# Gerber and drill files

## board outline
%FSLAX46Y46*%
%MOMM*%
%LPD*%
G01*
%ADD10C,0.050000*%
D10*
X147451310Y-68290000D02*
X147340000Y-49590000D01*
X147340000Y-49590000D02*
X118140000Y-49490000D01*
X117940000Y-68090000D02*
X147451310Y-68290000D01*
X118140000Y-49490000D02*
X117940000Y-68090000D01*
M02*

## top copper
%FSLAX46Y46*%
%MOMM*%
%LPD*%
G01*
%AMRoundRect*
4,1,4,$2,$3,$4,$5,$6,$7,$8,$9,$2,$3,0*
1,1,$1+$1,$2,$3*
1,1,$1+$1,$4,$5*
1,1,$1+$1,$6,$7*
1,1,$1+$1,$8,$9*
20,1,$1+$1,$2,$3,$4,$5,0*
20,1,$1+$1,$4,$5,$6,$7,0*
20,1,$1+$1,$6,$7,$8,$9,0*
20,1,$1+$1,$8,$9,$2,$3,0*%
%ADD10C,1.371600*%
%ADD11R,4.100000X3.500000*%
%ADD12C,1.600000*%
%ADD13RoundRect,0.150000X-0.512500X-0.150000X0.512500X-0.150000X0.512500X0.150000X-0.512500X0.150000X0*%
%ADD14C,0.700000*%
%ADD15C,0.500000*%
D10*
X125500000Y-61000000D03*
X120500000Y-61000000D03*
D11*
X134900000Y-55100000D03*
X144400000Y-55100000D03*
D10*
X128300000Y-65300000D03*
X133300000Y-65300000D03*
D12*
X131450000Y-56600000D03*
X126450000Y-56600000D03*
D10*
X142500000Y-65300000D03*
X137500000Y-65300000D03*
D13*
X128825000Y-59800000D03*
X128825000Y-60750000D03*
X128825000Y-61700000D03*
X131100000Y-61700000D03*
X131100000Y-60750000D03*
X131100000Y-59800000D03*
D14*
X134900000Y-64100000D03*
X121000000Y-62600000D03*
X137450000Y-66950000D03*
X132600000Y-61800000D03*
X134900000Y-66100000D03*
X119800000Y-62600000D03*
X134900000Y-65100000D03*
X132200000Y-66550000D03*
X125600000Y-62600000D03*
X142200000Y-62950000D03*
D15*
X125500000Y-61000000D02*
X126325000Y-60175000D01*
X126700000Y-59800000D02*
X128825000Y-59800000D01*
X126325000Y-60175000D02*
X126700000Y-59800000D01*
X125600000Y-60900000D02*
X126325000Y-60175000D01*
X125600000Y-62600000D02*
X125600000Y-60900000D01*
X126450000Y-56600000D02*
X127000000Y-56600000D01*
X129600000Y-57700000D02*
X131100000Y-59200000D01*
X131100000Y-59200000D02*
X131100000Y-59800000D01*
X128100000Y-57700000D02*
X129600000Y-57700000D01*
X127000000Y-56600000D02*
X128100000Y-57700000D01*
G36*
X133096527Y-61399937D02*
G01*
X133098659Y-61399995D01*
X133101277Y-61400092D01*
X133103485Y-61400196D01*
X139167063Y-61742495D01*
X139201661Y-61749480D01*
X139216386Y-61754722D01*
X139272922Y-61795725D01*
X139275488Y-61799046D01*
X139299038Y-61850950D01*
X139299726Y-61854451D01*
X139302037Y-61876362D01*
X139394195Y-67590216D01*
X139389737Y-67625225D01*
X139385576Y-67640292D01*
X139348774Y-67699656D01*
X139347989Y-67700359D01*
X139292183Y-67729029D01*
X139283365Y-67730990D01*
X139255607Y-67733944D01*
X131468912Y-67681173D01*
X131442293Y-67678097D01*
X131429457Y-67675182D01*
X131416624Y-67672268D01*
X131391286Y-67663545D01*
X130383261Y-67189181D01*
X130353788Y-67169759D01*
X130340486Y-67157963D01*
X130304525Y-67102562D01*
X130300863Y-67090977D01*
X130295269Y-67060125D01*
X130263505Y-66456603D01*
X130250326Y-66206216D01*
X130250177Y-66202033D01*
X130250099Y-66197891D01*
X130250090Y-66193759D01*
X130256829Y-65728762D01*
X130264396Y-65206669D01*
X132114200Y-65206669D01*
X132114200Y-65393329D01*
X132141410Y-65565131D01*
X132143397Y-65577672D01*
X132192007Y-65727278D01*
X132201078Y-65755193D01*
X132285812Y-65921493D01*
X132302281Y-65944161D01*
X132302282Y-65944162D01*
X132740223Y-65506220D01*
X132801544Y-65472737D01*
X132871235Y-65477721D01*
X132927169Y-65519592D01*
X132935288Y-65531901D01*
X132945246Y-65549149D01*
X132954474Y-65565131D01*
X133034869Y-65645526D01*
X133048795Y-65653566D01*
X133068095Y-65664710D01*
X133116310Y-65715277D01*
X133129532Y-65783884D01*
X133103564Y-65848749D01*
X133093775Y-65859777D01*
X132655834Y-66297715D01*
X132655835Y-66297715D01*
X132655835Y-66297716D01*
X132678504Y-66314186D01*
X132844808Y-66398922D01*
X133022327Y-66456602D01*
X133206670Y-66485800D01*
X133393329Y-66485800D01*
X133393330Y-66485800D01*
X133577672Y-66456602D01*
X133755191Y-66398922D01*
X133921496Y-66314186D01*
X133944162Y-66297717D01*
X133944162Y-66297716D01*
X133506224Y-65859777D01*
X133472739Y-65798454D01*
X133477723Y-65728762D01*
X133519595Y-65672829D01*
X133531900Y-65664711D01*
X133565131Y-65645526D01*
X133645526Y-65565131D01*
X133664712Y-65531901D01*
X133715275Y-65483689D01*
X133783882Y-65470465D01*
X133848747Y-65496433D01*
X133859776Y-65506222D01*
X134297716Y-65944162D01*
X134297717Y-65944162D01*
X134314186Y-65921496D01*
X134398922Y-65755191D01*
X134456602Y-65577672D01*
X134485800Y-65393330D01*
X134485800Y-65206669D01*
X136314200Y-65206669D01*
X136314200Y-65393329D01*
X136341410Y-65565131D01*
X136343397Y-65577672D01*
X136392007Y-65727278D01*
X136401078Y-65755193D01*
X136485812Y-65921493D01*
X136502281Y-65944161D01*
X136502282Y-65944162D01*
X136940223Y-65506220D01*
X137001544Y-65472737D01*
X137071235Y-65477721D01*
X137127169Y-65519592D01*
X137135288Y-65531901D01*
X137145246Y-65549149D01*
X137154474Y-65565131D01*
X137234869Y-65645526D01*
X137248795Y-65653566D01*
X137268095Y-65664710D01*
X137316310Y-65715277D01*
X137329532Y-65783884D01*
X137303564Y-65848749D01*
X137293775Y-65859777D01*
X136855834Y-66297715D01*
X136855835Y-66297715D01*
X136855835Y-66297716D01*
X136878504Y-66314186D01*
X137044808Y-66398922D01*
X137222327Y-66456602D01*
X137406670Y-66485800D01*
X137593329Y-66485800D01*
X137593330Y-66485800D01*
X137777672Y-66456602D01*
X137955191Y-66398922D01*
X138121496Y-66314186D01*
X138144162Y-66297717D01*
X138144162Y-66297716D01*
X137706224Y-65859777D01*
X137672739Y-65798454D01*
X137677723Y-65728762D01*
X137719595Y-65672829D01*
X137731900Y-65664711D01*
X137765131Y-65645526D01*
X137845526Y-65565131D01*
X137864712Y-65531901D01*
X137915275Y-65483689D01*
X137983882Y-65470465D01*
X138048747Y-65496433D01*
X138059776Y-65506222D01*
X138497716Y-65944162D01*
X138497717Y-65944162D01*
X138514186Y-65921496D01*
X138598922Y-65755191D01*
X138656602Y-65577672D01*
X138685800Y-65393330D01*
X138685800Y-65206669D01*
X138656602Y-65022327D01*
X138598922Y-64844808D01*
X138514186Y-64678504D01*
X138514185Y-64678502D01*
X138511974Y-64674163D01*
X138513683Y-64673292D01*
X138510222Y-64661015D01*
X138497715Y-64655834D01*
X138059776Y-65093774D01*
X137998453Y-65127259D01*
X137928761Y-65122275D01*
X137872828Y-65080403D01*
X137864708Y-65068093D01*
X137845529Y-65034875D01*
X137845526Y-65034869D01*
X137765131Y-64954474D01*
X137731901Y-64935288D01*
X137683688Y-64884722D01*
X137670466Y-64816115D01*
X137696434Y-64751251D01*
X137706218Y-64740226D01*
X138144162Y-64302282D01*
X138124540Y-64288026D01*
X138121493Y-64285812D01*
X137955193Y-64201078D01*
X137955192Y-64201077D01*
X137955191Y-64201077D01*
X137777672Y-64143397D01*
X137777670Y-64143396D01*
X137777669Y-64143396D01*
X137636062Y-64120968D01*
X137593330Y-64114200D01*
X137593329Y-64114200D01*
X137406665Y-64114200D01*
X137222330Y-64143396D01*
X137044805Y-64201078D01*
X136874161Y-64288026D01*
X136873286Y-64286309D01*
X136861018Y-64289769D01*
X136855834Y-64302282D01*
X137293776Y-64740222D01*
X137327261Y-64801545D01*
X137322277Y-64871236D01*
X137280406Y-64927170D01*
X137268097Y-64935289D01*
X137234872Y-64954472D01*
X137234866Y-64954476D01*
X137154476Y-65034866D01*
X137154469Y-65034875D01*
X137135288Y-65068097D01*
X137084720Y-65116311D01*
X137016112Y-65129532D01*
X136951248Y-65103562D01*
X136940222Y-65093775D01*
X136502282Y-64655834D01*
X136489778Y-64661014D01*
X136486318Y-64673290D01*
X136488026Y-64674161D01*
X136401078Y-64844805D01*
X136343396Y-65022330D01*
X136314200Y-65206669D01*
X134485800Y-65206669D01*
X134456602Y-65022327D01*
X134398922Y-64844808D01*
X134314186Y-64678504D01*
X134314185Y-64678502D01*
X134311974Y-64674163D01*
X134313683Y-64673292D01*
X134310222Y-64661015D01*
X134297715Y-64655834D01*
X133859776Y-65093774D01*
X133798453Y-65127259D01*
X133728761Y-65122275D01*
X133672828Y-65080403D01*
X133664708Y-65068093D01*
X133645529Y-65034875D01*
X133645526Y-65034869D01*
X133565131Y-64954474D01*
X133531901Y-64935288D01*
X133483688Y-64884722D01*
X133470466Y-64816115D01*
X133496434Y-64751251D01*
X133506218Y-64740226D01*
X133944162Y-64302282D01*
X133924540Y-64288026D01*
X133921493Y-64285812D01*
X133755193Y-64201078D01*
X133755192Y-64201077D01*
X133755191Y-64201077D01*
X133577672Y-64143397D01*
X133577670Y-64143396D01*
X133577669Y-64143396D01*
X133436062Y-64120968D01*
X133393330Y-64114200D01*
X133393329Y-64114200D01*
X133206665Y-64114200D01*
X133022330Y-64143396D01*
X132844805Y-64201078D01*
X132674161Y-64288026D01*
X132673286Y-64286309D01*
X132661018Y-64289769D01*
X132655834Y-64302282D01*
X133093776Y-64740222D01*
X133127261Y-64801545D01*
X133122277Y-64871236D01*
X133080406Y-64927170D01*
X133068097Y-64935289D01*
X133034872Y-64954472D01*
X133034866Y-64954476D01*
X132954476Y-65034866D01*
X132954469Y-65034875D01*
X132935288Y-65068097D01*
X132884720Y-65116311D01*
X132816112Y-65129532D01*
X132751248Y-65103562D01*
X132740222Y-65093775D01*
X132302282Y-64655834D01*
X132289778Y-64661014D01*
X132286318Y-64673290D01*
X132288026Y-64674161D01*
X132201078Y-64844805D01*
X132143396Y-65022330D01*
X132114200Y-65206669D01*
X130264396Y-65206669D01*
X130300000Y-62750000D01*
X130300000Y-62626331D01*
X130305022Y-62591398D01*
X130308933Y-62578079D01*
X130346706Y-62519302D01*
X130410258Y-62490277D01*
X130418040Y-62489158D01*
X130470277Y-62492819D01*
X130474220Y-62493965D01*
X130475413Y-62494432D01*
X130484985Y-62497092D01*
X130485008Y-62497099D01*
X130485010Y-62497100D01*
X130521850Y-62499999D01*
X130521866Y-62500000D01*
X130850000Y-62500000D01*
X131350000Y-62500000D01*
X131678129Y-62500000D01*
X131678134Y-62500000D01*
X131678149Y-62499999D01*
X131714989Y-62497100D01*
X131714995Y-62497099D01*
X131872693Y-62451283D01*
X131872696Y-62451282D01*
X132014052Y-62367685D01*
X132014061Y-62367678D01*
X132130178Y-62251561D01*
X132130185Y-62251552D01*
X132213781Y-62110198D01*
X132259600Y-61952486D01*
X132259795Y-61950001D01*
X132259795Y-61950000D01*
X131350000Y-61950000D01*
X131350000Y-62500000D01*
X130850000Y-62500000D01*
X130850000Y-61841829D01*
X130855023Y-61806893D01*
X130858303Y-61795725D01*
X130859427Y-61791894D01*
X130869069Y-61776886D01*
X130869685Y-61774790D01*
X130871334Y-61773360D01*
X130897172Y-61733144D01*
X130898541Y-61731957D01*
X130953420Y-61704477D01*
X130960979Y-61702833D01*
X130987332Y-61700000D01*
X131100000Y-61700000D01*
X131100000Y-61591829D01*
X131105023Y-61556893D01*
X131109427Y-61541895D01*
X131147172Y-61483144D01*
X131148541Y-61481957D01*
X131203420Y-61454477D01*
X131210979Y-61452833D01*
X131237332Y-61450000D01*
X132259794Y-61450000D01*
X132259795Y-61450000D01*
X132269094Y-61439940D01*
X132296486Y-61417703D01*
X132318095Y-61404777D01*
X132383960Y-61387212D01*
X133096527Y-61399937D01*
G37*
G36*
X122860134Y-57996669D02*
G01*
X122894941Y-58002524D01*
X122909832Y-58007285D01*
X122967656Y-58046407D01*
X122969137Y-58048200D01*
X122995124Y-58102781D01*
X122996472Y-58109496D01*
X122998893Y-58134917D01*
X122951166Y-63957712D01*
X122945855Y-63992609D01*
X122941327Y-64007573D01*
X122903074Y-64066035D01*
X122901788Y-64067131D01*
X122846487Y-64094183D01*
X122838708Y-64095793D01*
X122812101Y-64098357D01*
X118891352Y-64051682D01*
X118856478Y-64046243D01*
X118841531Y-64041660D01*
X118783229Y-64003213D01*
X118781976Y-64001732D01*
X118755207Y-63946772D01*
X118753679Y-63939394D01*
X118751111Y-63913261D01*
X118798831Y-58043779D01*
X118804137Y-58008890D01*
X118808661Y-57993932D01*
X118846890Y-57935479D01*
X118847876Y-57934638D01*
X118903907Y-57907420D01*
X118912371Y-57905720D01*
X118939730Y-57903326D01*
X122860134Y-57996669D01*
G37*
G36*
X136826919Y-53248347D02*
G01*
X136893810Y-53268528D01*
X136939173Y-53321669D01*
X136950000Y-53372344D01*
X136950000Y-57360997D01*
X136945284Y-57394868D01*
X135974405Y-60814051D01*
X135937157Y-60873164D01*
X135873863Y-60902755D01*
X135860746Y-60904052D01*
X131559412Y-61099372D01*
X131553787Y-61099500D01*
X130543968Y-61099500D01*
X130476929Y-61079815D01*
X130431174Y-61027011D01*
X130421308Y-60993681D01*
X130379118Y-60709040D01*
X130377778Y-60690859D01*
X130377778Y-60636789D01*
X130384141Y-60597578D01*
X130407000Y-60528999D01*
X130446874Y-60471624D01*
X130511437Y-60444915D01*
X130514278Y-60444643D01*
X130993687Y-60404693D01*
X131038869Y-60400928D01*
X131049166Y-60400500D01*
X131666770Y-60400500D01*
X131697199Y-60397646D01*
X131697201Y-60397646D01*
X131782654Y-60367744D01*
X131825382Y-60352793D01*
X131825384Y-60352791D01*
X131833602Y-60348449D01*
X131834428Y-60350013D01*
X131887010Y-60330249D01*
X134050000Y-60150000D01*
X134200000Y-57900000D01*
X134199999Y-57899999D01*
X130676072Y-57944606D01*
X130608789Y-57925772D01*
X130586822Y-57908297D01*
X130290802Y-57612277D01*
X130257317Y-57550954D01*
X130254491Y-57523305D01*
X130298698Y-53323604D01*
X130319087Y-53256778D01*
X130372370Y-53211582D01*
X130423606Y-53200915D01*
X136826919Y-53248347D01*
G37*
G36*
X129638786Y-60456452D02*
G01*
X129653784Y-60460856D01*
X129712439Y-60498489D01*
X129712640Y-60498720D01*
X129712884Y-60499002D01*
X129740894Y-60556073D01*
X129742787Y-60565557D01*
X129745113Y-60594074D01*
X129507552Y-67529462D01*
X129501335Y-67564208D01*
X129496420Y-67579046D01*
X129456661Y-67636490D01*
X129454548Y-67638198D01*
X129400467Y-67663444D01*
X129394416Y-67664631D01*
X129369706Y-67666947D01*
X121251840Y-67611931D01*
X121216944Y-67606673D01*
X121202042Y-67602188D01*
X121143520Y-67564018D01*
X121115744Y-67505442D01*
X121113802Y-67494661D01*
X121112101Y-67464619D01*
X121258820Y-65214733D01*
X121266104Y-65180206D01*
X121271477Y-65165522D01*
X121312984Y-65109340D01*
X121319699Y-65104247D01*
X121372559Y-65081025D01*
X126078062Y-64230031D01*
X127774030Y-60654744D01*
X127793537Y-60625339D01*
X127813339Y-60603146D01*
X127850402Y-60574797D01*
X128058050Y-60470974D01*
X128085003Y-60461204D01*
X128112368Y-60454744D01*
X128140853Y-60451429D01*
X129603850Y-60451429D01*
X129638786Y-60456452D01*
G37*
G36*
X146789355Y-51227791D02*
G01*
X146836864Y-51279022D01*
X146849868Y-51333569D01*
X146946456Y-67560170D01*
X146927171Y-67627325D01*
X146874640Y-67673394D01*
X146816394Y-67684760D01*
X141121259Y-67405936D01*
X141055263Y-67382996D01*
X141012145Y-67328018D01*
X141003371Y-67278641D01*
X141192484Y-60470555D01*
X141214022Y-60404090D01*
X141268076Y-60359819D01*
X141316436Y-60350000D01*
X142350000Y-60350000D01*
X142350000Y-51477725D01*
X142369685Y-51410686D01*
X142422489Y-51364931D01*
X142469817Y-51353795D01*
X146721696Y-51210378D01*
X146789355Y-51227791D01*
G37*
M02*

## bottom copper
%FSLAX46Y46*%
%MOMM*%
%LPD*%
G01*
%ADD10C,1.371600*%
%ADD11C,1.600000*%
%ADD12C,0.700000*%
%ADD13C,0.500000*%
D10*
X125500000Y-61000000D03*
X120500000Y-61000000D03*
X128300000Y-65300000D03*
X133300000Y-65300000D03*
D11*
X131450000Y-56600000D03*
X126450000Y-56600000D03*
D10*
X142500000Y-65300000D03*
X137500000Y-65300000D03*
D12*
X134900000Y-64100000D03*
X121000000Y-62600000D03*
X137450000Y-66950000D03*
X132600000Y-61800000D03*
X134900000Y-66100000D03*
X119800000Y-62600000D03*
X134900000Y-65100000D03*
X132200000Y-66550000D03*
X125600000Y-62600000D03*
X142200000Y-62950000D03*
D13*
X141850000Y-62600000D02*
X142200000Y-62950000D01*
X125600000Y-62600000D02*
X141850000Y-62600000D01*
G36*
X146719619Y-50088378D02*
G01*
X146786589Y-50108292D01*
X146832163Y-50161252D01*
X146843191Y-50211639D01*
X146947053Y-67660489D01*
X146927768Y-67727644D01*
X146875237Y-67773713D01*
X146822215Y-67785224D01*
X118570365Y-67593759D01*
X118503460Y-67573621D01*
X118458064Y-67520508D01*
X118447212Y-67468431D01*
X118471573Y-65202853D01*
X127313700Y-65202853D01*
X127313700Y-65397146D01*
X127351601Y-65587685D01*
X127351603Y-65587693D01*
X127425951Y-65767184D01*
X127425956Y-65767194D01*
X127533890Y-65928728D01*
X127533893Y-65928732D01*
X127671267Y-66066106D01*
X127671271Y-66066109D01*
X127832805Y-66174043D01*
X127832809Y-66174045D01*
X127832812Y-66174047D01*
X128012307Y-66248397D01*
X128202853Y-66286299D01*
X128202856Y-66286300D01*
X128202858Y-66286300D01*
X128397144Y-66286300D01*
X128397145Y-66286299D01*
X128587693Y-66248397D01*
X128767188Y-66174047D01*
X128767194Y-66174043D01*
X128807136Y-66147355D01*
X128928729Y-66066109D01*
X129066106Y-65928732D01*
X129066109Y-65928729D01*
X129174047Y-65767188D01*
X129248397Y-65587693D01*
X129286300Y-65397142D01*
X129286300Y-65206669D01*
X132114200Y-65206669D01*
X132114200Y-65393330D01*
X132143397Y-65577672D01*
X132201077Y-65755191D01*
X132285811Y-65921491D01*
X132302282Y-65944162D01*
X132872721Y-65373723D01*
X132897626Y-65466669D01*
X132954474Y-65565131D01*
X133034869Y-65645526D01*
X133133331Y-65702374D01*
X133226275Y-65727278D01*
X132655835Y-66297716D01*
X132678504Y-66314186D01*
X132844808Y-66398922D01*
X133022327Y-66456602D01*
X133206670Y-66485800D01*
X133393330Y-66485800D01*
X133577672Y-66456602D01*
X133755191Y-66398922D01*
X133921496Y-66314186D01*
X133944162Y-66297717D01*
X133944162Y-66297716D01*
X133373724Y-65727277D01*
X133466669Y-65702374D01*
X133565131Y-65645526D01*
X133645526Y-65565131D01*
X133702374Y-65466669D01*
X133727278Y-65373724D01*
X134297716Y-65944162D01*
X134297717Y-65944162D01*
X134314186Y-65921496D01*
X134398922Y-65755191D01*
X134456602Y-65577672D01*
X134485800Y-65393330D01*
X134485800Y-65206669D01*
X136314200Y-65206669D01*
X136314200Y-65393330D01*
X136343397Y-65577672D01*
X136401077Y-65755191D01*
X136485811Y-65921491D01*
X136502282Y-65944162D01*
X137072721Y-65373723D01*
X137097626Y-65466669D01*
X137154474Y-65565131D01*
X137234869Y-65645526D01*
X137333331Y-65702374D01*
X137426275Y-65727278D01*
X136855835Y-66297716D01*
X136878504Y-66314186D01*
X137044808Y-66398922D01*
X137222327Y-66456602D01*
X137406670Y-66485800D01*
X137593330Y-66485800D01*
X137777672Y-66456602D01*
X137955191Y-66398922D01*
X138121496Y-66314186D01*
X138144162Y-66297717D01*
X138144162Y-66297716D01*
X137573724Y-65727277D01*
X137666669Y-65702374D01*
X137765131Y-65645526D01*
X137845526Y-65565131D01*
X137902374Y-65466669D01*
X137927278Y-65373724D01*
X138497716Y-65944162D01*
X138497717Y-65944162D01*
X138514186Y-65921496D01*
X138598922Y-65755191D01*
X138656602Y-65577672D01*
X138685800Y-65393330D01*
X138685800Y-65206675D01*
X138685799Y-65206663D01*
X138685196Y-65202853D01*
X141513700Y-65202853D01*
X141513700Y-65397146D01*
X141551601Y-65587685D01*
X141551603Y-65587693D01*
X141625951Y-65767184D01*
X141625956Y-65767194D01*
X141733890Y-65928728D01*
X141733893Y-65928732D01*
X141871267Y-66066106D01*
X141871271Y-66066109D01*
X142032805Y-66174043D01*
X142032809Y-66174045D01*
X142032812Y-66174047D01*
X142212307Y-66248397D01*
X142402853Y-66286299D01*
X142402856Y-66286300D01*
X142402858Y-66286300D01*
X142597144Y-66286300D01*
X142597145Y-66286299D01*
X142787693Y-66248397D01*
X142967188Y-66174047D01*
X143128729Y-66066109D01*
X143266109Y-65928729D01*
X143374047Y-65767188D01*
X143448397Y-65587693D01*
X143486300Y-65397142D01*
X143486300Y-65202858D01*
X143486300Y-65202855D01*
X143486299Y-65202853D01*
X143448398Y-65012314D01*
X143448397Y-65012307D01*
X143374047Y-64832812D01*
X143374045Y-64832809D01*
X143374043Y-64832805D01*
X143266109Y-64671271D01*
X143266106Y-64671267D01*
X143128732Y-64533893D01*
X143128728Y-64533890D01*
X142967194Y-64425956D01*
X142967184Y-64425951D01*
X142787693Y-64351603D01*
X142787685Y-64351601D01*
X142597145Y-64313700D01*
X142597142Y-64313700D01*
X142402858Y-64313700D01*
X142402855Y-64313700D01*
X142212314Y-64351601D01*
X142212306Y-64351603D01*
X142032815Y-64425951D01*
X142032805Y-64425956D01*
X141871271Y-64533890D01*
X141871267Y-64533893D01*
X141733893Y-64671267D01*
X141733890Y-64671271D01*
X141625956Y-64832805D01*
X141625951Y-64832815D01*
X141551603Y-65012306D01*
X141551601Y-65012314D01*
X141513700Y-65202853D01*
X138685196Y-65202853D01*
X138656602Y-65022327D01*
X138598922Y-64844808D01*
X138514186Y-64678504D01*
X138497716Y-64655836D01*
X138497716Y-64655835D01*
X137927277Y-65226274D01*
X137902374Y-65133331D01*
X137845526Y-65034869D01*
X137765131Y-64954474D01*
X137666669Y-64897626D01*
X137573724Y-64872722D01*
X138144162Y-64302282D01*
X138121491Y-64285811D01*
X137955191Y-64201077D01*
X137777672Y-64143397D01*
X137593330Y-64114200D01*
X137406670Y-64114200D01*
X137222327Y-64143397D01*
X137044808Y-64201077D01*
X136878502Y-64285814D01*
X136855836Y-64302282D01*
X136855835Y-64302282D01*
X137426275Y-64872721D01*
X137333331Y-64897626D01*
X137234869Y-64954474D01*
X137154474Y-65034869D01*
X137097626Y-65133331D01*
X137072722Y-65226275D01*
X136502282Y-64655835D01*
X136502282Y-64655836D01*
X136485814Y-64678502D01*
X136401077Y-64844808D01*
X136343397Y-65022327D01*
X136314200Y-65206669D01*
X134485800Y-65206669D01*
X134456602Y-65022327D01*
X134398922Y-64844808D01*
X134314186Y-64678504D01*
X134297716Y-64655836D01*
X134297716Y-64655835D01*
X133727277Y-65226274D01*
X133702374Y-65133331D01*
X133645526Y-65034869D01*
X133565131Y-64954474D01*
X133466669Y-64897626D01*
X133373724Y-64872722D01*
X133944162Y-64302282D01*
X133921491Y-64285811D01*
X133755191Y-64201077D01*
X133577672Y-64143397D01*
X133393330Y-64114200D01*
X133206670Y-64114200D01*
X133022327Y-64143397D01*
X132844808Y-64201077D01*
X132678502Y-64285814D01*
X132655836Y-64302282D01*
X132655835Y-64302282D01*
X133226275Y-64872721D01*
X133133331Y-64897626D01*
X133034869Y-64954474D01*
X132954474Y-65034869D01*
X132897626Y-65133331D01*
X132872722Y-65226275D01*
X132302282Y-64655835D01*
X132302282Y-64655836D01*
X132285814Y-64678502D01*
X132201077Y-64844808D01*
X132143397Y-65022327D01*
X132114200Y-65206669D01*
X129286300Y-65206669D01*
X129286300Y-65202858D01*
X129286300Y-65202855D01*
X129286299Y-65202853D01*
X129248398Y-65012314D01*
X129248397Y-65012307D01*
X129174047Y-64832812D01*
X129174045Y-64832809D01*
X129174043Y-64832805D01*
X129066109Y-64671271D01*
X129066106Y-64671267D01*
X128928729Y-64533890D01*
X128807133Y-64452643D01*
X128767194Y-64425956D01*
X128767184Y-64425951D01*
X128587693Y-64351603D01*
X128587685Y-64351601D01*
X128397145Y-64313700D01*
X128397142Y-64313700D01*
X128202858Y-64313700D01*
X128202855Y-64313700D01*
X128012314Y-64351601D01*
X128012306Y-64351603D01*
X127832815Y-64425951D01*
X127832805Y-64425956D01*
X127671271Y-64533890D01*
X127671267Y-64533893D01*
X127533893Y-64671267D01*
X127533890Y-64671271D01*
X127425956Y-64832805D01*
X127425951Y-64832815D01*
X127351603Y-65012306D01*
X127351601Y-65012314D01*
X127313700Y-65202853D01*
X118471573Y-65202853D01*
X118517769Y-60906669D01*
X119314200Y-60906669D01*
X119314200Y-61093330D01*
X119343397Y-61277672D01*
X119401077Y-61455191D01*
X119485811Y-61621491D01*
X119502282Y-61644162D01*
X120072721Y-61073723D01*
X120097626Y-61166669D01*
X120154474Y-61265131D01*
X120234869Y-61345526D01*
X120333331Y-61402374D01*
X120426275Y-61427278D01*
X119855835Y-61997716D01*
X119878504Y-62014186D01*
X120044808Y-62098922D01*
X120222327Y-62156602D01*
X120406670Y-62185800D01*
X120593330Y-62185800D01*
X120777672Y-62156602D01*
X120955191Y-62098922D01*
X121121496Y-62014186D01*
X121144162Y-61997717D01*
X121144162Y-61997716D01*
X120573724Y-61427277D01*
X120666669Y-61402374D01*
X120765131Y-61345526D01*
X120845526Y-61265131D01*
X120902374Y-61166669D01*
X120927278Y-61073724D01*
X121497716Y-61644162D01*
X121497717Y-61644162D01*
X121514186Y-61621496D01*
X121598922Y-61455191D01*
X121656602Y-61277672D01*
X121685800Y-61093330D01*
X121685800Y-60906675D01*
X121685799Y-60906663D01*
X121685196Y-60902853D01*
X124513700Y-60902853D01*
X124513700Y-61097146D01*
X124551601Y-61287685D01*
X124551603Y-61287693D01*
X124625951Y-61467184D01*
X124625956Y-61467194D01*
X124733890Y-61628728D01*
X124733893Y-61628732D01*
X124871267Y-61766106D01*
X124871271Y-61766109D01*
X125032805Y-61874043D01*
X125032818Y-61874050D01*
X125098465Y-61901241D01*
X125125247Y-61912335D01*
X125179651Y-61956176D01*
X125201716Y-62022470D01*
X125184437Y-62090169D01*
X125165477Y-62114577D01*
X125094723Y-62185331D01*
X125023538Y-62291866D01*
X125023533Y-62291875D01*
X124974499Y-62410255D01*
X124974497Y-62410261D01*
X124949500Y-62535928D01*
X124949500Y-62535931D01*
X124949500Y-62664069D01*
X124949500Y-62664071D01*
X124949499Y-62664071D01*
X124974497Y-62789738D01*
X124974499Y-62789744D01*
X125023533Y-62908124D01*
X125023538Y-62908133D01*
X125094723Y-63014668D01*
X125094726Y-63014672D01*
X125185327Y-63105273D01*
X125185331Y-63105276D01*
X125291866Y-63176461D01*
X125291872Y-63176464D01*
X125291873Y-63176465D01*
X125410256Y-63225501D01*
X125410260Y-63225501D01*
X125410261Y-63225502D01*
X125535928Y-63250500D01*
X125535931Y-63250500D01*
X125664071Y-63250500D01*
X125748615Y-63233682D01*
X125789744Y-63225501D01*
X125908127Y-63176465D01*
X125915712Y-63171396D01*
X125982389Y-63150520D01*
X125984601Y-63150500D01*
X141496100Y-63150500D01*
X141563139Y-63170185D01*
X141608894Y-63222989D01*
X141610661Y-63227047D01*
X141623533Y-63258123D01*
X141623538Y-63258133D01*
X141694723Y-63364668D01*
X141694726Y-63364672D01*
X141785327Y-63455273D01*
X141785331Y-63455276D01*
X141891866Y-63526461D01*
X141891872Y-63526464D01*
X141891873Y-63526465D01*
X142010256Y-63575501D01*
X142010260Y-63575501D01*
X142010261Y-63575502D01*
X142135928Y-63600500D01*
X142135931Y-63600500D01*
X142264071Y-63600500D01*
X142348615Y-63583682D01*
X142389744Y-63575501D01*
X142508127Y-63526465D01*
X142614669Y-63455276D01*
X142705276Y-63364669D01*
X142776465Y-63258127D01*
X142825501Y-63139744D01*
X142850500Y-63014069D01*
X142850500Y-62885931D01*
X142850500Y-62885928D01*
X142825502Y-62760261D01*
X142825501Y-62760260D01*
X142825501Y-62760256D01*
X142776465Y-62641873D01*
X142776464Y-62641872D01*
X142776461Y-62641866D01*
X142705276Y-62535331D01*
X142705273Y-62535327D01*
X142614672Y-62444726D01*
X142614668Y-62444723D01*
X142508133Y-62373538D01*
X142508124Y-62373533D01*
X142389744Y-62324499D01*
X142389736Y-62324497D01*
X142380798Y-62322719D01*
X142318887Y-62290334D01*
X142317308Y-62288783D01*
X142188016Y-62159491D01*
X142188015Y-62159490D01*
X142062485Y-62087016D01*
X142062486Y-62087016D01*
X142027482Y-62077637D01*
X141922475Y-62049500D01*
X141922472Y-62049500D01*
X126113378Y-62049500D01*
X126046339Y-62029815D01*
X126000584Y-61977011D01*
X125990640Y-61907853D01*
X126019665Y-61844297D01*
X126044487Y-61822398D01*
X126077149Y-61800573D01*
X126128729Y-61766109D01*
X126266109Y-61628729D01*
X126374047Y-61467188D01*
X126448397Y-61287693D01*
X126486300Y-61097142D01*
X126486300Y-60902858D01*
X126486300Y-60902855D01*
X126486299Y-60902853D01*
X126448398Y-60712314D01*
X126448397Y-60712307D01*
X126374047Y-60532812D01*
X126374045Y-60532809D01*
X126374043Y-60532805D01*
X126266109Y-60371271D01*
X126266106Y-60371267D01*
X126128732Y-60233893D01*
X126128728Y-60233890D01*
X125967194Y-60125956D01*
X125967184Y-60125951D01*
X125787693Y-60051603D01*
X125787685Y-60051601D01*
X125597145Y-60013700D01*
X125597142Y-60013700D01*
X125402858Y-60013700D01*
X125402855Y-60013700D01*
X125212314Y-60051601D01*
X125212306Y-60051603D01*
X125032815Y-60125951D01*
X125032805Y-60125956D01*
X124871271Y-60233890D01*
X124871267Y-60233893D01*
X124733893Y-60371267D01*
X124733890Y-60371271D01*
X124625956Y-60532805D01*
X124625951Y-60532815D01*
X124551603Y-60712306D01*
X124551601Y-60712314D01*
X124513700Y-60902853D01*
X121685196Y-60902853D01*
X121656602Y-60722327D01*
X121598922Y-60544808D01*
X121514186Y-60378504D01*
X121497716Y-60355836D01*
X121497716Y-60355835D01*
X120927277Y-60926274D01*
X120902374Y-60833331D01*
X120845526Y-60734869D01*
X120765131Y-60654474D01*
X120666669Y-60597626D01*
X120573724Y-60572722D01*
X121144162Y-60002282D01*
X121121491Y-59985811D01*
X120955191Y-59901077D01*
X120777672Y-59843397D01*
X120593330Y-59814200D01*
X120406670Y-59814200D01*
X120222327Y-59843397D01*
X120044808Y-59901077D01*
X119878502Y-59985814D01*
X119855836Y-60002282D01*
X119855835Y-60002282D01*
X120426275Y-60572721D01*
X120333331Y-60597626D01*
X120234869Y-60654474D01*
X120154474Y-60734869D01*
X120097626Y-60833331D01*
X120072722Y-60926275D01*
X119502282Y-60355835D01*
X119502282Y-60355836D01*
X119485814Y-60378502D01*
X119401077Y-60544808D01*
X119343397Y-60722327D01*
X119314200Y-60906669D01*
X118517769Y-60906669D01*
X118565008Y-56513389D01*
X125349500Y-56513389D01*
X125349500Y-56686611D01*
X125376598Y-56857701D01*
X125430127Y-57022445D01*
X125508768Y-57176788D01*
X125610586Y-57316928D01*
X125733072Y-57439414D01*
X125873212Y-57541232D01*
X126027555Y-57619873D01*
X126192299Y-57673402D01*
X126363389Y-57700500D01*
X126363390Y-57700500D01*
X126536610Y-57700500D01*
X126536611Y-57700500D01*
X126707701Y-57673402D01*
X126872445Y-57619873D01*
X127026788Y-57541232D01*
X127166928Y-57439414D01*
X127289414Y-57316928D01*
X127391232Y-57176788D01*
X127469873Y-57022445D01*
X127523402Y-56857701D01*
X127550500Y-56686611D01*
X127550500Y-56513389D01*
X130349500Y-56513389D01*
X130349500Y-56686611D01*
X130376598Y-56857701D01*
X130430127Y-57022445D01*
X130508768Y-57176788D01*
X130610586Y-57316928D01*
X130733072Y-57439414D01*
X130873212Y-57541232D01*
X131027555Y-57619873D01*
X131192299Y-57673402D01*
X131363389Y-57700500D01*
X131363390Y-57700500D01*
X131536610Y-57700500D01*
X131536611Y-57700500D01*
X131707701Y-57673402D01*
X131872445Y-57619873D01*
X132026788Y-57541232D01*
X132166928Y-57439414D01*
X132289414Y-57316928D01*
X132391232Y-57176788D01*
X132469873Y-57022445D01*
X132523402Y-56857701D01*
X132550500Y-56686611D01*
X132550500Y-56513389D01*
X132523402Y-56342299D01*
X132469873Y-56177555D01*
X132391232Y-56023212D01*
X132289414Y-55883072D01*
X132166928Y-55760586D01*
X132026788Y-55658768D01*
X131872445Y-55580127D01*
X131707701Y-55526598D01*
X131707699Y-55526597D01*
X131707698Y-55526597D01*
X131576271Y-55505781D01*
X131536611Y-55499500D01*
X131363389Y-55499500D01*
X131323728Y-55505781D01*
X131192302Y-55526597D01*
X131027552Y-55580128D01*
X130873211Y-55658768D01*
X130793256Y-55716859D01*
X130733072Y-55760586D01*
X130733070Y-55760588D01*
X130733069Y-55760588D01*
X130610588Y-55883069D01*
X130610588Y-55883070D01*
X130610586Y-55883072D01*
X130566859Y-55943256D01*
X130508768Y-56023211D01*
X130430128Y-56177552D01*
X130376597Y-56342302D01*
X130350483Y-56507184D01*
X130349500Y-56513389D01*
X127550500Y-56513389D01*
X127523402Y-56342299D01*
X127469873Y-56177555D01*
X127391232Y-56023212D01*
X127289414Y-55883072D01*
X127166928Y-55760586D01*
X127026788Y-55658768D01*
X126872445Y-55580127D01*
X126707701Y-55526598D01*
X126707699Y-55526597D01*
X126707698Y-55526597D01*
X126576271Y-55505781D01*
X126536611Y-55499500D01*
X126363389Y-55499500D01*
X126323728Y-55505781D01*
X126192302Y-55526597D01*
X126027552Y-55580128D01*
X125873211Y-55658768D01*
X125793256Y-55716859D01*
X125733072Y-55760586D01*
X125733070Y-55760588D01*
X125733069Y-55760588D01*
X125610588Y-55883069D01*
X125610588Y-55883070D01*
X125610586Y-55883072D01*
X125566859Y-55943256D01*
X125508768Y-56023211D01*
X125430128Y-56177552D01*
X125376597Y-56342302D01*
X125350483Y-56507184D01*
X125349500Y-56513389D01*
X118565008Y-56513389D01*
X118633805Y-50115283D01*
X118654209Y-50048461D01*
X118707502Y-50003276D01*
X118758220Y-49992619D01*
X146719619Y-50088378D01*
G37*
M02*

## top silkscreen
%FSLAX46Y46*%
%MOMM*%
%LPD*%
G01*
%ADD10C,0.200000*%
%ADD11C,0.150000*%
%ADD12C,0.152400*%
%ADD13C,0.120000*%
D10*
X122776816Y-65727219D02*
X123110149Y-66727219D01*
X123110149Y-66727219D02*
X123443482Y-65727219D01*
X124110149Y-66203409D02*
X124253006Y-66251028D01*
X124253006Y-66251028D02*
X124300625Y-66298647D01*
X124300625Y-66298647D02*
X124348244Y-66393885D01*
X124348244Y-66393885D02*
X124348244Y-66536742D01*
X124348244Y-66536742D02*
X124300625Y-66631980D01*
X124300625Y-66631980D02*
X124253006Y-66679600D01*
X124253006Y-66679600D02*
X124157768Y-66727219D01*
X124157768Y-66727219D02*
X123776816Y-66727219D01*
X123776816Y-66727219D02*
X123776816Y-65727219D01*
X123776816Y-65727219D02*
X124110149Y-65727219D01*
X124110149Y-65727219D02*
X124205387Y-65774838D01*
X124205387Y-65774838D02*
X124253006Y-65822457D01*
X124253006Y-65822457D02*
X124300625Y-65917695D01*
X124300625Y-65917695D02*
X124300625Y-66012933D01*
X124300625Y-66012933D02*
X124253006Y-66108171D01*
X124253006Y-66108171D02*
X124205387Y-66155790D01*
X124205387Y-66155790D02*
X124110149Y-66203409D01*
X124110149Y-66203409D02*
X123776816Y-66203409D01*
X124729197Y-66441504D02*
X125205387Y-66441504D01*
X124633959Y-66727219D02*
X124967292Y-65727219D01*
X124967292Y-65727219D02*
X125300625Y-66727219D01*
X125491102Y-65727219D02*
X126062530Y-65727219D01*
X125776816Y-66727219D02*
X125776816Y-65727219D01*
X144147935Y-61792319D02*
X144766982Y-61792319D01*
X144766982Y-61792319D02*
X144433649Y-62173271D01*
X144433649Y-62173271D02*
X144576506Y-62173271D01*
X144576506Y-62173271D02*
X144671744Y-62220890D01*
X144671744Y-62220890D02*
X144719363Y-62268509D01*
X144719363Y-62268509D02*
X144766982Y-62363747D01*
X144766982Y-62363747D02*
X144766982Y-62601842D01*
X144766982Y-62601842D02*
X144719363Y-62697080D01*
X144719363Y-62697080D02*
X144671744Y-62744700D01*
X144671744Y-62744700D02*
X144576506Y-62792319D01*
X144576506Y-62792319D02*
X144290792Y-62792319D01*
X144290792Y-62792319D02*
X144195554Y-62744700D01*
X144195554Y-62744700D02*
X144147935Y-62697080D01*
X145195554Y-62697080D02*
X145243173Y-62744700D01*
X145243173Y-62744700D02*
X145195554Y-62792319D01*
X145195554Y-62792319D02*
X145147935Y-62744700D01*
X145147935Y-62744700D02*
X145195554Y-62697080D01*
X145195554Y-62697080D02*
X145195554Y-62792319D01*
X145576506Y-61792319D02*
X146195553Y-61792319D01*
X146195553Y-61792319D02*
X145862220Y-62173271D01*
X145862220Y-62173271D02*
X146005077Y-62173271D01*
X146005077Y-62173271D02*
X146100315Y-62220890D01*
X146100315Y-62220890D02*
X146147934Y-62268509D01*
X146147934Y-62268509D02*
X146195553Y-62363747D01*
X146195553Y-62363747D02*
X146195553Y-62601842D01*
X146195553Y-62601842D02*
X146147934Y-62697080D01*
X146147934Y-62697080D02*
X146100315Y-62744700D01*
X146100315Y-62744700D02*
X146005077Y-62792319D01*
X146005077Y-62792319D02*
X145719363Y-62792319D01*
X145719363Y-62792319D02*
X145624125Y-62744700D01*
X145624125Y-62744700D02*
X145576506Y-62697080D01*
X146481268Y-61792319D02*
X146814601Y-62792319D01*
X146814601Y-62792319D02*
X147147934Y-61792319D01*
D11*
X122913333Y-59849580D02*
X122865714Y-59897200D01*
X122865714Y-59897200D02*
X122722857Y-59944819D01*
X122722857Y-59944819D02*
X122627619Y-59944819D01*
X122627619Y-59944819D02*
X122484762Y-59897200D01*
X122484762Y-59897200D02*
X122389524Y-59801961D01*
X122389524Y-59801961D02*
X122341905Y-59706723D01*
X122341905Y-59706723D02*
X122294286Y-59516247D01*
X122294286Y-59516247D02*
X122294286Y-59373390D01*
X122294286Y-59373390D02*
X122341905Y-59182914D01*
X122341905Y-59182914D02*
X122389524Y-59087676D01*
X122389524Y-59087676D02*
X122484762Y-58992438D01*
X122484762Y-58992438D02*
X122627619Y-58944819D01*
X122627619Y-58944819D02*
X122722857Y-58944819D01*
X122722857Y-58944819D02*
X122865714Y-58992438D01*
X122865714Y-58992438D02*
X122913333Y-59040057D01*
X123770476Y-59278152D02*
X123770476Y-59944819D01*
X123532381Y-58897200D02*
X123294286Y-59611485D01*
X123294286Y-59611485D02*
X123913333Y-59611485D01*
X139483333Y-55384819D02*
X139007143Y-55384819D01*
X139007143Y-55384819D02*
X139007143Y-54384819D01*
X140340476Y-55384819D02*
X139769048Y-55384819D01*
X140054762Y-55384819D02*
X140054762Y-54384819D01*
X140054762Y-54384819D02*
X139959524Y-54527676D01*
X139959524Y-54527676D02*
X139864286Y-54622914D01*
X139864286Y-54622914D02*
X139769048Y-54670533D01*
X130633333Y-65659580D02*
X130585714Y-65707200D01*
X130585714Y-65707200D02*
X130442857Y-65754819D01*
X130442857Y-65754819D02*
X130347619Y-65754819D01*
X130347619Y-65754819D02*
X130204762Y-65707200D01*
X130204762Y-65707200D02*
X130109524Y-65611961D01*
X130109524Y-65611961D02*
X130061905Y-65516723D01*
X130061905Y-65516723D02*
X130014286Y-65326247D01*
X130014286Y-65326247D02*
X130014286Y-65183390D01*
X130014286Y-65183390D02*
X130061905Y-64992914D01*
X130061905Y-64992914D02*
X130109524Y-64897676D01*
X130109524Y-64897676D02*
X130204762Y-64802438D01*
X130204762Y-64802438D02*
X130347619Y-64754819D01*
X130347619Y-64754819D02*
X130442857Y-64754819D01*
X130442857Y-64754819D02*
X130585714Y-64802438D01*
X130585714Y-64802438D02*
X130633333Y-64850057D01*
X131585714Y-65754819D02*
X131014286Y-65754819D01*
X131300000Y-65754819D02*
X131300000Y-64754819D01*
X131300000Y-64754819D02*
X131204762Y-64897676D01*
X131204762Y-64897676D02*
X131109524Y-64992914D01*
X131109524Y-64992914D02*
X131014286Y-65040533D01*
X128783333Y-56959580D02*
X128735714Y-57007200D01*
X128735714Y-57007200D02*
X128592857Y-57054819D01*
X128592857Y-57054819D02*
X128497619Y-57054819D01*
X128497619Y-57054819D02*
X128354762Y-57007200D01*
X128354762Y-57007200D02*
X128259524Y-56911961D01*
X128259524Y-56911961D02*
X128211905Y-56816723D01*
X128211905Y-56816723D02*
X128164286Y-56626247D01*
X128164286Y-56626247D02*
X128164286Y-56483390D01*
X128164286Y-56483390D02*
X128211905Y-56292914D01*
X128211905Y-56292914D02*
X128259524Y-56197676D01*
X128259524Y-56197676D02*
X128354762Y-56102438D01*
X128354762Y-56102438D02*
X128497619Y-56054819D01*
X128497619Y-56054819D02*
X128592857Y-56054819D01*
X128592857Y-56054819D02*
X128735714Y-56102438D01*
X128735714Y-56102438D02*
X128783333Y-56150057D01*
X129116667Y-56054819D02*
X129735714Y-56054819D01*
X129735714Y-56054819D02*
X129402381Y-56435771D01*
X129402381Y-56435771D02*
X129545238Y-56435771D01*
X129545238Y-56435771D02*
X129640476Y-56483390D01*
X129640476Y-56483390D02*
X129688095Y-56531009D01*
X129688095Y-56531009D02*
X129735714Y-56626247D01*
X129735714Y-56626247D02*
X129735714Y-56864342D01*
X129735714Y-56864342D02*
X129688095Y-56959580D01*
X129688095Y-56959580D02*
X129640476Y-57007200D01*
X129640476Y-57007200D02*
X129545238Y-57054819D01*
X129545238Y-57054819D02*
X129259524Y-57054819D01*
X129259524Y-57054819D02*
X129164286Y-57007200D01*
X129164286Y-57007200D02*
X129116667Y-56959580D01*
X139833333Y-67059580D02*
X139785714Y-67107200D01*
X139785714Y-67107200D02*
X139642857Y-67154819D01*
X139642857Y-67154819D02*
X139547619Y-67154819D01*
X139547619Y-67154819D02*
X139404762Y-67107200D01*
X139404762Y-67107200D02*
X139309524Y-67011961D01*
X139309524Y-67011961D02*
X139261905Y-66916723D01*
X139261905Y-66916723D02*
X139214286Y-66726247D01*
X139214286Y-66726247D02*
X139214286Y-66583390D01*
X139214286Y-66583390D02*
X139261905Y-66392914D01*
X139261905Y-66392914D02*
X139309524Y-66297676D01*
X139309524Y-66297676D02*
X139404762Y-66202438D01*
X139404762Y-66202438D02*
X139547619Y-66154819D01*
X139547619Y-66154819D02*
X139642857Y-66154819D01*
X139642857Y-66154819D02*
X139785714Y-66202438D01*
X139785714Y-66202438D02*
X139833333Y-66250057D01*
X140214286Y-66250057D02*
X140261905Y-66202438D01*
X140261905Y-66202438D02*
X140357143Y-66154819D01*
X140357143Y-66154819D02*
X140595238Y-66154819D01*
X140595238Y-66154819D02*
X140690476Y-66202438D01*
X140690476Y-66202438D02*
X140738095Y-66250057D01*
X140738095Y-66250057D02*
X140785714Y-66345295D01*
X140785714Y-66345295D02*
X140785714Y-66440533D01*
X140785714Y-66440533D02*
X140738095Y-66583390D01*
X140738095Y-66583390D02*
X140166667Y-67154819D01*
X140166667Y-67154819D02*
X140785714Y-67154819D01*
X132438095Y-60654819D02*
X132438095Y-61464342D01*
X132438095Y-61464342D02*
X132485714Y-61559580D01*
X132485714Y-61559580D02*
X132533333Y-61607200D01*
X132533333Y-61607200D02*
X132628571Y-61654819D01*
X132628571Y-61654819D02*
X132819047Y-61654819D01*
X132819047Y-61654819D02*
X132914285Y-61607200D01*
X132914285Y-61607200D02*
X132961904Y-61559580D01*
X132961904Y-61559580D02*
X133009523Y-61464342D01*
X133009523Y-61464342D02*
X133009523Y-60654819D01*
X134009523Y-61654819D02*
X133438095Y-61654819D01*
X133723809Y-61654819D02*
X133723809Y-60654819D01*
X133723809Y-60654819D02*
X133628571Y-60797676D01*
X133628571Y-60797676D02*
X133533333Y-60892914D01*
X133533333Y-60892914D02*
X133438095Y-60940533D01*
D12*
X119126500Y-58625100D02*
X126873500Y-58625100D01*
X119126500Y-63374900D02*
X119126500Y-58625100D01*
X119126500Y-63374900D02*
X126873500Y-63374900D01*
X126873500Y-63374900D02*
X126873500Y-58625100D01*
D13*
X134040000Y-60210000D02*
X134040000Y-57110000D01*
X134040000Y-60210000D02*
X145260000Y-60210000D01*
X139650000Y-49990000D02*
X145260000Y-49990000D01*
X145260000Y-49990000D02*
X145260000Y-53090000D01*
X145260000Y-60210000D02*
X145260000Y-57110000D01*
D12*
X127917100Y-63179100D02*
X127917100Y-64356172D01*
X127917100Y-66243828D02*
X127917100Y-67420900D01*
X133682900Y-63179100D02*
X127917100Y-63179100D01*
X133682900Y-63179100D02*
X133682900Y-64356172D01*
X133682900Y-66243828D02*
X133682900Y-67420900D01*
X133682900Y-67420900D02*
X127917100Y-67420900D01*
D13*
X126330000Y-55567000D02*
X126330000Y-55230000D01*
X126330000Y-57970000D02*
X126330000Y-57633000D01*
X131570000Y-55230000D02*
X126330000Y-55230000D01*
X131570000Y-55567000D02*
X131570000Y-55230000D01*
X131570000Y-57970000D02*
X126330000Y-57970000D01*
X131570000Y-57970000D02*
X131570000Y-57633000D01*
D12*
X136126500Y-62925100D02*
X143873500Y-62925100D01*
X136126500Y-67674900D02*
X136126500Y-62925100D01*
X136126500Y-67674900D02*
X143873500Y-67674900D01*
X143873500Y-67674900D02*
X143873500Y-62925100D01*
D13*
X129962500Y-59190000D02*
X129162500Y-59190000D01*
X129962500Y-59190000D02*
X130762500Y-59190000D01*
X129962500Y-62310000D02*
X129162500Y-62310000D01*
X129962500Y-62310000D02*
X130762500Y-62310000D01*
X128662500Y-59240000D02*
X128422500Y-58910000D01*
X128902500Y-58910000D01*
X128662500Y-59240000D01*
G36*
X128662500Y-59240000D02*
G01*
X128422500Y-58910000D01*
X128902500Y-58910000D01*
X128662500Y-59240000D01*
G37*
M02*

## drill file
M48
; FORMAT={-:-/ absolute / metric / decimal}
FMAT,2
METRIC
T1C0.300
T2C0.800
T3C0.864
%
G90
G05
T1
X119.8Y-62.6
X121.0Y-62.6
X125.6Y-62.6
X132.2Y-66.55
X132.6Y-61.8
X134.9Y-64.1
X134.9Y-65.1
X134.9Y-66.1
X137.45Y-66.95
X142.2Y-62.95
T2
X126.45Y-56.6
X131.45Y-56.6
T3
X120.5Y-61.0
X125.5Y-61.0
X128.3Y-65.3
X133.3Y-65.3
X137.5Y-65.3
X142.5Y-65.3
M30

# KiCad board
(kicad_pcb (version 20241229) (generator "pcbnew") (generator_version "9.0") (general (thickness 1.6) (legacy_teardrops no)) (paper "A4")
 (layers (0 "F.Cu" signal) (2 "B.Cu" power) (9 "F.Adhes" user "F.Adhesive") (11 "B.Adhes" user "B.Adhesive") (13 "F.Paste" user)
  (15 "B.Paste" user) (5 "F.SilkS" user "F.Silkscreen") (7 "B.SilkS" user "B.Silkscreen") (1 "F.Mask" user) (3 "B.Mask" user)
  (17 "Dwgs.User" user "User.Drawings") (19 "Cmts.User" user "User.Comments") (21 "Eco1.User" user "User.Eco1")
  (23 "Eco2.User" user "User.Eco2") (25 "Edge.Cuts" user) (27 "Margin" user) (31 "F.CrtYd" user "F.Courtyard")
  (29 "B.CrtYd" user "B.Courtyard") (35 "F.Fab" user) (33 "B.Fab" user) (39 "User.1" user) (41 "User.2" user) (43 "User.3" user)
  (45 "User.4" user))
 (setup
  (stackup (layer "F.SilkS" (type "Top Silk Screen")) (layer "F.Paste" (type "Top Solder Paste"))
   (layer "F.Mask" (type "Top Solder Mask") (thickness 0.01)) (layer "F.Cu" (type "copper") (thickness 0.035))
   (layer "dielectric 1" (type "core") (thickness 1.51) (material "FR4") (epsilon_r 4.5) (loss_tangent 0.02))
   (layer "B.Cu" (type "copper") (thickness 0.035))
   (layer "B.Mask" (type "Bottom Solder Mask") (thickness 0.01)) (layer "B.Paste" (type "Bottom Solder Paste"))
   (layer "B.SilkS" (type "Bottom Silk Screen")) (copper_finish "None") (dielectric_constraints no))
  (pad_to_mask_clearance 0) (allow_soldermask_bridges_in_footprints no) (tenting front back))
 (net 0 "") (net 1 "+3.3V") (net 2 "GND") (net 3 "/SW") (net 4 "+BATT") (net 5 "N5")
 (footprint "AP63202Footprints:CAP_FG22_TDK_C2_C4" (layer "F.Cu") (at 125.5 61 180)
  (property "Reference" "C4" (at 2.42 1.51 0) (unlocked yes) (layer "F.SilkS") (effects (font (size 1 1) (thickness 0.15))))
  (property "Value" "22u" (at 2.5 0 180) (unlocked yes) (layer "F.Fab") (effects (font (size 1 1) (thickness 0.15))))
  (fp_line (start 6.3735 2.3749) (end -1.3735 2.3749) (stroke (width 0.1524) (type solid)) (layer "F.SilkS"))
  (fp_line (start 6.3735 -2.3749) (end 6.3735 2.3749) (stroke (width 0.1524) (type solid)) (layer "F.SilkS"))
  (fp_line (start 6.3735 -2.3749) (end -1.3735 -2.3749) (stroke (width 0.1524) (type solid)) (layer "F.SilkS"))
  (fp_line (start -1.3735 -2.3749) (end -1.3735 2.3749) (stroke (width 0.1524) (type solid)) (layer "F.SilkS"))
  (pad "1" thru_hole circle (at 0 0 180) (size 1.3716 1.3716) (drill 0.8636) (layers "*.Cu" "*.Mask") (remove_unused_layers no)
   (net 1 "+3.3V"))
  (pad "2" thru_hole circle (at 5 0 180) (size 1.3716 1.3716) (drill 0.8636) (layers "*.Cu" "*.Mask") (remove_unused_layers no)
   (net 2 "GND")))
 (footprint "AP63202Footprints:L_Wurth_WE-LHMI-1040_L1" (layer "F.Cu") (at 139.65 55.1)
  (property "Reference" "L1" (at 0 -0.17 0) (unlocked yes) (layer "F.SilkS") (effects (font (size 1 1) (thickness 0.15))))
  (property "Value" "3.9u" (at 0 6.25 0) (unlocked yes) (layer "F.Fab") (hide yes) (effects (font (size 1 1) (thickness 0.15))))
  (fp_line (start -5.61 5.11) (end -5.61 2.01) (stroke (width 0.12) (type solid)) (layer "F.SilkS"))
  (fp_line (start -5.61 5.11) (end 5.61 5.11) (stroke (width 0.12) (type solid)) (layer "F.SilkS"))
  (fp_line (start 0 -5.11) (end 5.61 -5.11) (stroke (width 0.12) (type solid)) (layer "F.SilkS"))
  (fp_line (start 5.61 -5.11) (end 5.61 -2.01) (stroke (width 0.12) (type solid)) (layer "F.SilkS"))
  (fp_line (start 5.61 5.11) (end 5.61 2.01) (stroke (width 0.12) (type solid)) (layer "F.SilkS"))
  (pad "1" smd rect (at -4.75 0) (size 4.1 3.5) (layers "F.Cu" "F.Mask" "F.Paste") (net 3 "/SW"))
  (pad "2" smd rect (at 4.75 0) (size 4.1 3.5) (layers "F.Cu" "F.Mask" "F.Paste") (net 1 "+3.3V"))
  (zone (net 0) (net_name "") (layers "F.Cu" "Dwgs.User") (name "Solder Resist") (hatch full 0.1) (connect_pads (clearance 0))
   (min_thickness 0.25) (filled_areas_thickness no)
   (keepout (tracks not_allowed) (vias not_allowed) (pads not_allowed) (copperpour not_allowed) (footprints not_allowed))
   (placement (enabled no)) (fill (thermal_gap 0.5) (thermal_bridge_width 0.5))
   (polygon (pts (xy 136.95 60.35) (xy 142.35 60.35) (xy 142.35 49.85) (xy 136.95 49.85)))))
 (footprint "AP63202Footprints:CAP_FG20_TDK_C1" (layer "F.Cu") (at 128.3 65.3)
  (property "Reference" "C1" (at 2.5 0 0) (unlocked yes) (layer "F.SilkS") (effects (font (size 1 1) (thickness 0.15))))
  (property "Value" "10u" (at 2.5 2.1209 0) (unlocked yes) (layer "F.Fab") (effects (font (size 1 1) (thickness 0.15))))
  (fp_line (start -0.3829 -2.1209) (end -0.3829 -0.943828) (stroke (width 0.1524) (type solid)) (layer "F.SilkS"))
  (fp_line (start -0.3829 0.943828) (end -0.3829 2.1209) (stroke (width 0.1524) (type solid)) (layer "F.SilkS"))
  (fp_line (start 5.3829 -2.1209) (end -0.3829 -2.1209) (stroke (width 0.1524) (type solid)) (layer "F.SilkS"))
  (fp_line (start 5.3829 -2.1209) (end 5.3829 -0.943828) (stroke (width 0.1524) (type solid)) (layer "F.SilkS"))
  (fp_line (start 5.3829 0.943828) (end 5.3829 2.1209) (stroke (width 0.1524) (type solid)) (layer "F.SilkS"))
  (fp_line (start 5.3829 2.1209) (end -0.3829 2.1209) (stroke (width 0.1524) (type solid)) (layer "F.SilkS"))
  (pad "1" thru_hole circle (at 0 0) (size 1.3716 1.3716) (drill 0.8636) (layers "*.Cu" "*.Mask") (remove_unused_layers no) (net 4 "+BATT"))
  (pad "2" thru_hole circle (at 5 0) (size 1.3716 1.3716) (drill 0.8636) (layers "*.Cu" "*.Mask") (remove_unused_layers no) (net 2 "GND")))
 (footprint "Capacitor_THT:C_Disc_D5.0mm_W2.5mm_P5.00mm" (layer "F.Cu") (at 131.45 56.6 180)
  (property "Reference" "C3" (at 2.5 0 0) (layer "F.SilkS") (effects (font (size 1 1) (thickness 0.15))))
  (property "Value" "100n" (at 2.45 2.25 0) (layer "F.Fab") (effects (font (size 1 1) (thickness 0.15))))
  (fp_line (start 5.12 1.033) (end 5.12 1.37) (stroke (width 0.12) (type solid)) (layer "F.SilkS"))
  (fp_line (start 5.12 -1.37) (end 5.12 -1.033) (stroke (width 0.12) (type solid)) (layer "F.SilkS"))
  (fp_line (start -0.12 1.37) (end 5.12 1.37) (stroke (width 0.12) (type solid)) (layer "F.SilkS"))
  (fp_line (start -0.12 1.033) (end -0.12 1.37) (stroke (width 0.12) (type solid)) (layer "F.SilkS"))
  (fp_line (start -0.12 -1.37) (end 5.12 -1.37) (stroke (width 0.12) (type solid)) (layer "F.SilkS"))
  (fp_line (start -0.12 -1.37) (end -0.12 -1.033) (stroke (width 0.12) (type solid)) (layer "F.SilkS"))
  (pad "1" thru_hole circle (at 0 0 180) (size 1.6 1.6) (drill 0.8) (layers "*.Cu" "*.Mask") (remove_unused_layers no) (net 3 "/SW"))
  (pad "2" thru_hole circle (at 5 0 180) (size 1.6 1.6) (drill 0.8) (layers "*.Cu" "*.Mask") (remove_unused_layers no) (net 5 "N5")))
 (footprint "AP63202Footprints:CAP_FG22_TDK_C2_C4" (layer "F.Cu") (at 142.5 65.3 180)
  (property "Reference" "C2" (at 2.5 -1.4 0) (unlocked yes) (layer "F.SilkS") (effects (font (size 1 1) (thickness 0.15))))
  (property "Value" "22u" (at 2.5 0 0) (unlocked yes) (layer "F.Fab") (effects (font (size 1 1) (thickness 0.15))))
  (fp_line (start 6.3735 2.3749) (end -1.3735 2.3749) (stroke (width 0.1524) (type solid)) (layer "F.SilkS"))
  (fp_line (start 6.3735 -2.3749) (end 6.3735 2.3749) (stroke (width 0.1524) (type solid)) (layer "F.SilkS"))
  (fp_line (start 6.3735 -2.3749) (end -1.3735 -2.3749) (stroke (width 0.1524) (type solid)) (layer "F.SilkS"))
  (fp_line (start -1.3735 -2.3749) (end -1.3735 2.3749) (stroke (width 0.1524) (type solid)) (layer "F.SilkS"))
  (pad "1" thru_hole circle (at 0 0 180) (size 1.3716 1.3716) (drill 0.8636) (layers "*.Cu" "*.Mask") (remove_unused_layers no)
   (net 1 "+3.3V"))
  (pad "2" thru_hole circle (at 5 0 180) (size 1.3716 1.3716) (drill 0.8636) (layers "*.Cu" "*.Mask") (remove_unused_layers no)
   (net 2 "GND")))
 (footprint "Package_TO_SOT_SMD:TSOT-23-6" (layer "F.Cu") (at 129.9625 60.75)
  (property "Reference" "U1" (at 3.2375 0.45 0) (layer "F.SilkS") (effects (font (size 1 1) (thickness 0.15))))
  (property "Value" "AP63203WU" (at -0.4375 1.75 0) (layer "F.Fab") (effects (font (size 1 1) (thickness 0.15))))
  (fp_line (start 0 -1.56) (end -0.8 -1.56) (stroke (width 0.12) (type solid)) (layer "F.SilkS"))
  (fp_line (start 0 -1.56) (end 0.8 -1.56) (stroke (width 0.12) (type solid)) (layer "F.SilkS"))
  (fp_line (start 0 1.56) (end -0.8 1.56) (stroke (width 0.12) (type solid)) (layer "F.SilkS"))
  (fp_line (start 0 1.56) (end 0.8 1.56) (stroke (width 0.12) (type solid)) (layer "F.SilkS"))
  (fp_poly (pts (xy -1.3 -1.51) (xy -1.54 -1.84) (xy -1.06 -1.84)) (stroke (width 0.12) (type solid)) (fill yes) (layer "F.SilkS"))
  (pad "1" smd roundrect (at -1.1375 -0.95) (size 1.325 0.6) (layers "F.Cu" "F.Mask" "F.Paste") (roundrect_rratio 0.25) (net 1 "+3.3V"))
  (pad "2" smd roundrect (at -1.1375 0) (size 1.325 0.6) (layers "F.Cu" "F.Mask" "F.Paste") (roundrect_rratio 0.25) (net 4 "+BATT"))
  (pad "3" smd roundrect (at -1.1375 0.95) (size 1.325 0.6) (layers "F.Cu" "F.Mask" "F.Paste") (roundrect_rratio 0.25) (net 4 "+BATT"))
  (pad "4" smd roundrect (at 1.1375 0.95) (size 1.325 0.6) (layers "F.Cu" "F.Mask" "F.Paste") (roundrect_rratio 0.25) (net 2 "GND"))
  (pad "5" smd roundrect (at 1.1375 0) (size 1.325 0.6) (layers "F.Cu" "F.Mask" "F.Paste") (roundrect_rratio 0.25) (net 3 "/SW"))
  (pad "6" smd roundrect (at 1.1375 -0.95) (size 1.325 0.6) (layers "F.Cu" "F.Mask" "F.Paste") (roundrect_rratio 0.25) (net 5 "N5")))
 (gr_line (start 147.45131 68.29) (end 147.34 49.59) (stroke (width 0.05) (type default)) (layer "Edge.Cuts"))
 (gr_line (start 147.34 49.59) (end 118.14 49.49) (stroke (width 0.05) (type default)) (layer "Edge.Cuts"))
 (gr_line (start 117.94 68.09) (end 147.45131 68.29) (stroke (width 0.05) (type default)) (layer "Edge.Cuts"))
 (gr_line (start 118.14 49.49) (end 117.94 68.09) (stroke (width 0.05) (type default)) (layer "Edge.Cuts"))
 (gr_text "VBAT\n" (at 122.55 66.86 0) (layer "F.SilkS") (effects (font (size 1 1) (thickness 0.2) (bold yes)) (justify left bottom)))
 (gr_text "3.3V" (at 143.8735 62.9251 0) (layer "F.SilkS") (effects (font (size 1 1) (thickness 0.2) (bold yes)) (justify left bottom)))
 (via (at 134.9 64.1) (size 0.7) (drill 0.3) (layers "F.Cu" "B.Cu") (free yes) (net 2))
 (via (at 121 62.6) (size 0.7) (drill 0.3) (layers "F.Cu" "B.Cu") (free yes) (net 2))
 (via (at 137.45 66.95) (size 0.7) (drill 0.3) (layers "F.Cu" "B.Cu") (free yes) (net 2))
 (via (at 132.6 61.8) (size 0.7) (drill 0.3) (layers "F.Cu" "B.Cu") (free yes) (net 2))
 (via (at 134.9 66.1) (size 0.7) (drill 0.3) (layers "F.Cu" "B.Cu") (free yes) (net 2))
 (via (at 119.8 62.6) (size 0.7) (drill 0.3) (layers "F.Cu" "B.Cu") (free yes) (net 2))
 (via (at 134.9 65.1) (size 0.7) (drill 0.3) (layers "F.Cu" "B.Cu") (free yes) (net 2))
 (via (at 132.2 66.55) (size 0.7) (drill 0.3) (layers "F.Cu" "B.Cu") (free yes) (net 2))
 (segment (start 125.5 61) (end 126.325 60.175) (width 0.5) (layer "F.Cu") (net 1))
 (segment (start 126.7 59.8) (end 128.825 59.8) (width 0.5) (layer "F.Cu") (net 1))
 (segment (start 126.325 60.175) (end 126.7 59.8) (width 0.5) (layer "F.Cu") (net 1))
 (segment (start 125.6 60.9) (end 126.325 60.175) (width 0.5) (layer "F.Cu") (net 1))
 (segment (start 125.6 62.6) (end 125.6 60.9) (width 0.5) (layer "F.Cu") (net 1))
 (via (at 125.6 62.6) (size 0.7) (drill 0.3) (layers "F.Cu" "B.Cu") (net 1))
 (via (at 142.2 62.95) (size 0.7) (drill 0.3) (layers "F.Cu" "B.Cu") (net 1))
 (segment (start 141.85 62.6) (end 142.2 62.95) (width 0.5) (layer "B.Cu") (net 1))
 (segment (start 125.6 62.6) (end 141.85 62.6) (width 0.5) (layer "B.Cu") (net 1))
 (segment (start 126.45 56.6) (end 127 56.6) (width 0.5) (layer "F.Cu") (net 5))
 (segment (start 129.6 57.7) (end 131.1 59.2) (width 0.5) (layer "F.Cu") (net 5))
 (segment (start 131.1 59.2) (end 131.1 59.8) (width 0.5) (layer "F.Cu") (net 5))
 (segment (start 128.1 57.7) (end 129.6 57.7) (width 0.5) (layer "F.Cu") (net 5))
 (segment (start 127 56.6) (end 128.1 57.7) (width 0.5) (layer "F.Cu") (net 5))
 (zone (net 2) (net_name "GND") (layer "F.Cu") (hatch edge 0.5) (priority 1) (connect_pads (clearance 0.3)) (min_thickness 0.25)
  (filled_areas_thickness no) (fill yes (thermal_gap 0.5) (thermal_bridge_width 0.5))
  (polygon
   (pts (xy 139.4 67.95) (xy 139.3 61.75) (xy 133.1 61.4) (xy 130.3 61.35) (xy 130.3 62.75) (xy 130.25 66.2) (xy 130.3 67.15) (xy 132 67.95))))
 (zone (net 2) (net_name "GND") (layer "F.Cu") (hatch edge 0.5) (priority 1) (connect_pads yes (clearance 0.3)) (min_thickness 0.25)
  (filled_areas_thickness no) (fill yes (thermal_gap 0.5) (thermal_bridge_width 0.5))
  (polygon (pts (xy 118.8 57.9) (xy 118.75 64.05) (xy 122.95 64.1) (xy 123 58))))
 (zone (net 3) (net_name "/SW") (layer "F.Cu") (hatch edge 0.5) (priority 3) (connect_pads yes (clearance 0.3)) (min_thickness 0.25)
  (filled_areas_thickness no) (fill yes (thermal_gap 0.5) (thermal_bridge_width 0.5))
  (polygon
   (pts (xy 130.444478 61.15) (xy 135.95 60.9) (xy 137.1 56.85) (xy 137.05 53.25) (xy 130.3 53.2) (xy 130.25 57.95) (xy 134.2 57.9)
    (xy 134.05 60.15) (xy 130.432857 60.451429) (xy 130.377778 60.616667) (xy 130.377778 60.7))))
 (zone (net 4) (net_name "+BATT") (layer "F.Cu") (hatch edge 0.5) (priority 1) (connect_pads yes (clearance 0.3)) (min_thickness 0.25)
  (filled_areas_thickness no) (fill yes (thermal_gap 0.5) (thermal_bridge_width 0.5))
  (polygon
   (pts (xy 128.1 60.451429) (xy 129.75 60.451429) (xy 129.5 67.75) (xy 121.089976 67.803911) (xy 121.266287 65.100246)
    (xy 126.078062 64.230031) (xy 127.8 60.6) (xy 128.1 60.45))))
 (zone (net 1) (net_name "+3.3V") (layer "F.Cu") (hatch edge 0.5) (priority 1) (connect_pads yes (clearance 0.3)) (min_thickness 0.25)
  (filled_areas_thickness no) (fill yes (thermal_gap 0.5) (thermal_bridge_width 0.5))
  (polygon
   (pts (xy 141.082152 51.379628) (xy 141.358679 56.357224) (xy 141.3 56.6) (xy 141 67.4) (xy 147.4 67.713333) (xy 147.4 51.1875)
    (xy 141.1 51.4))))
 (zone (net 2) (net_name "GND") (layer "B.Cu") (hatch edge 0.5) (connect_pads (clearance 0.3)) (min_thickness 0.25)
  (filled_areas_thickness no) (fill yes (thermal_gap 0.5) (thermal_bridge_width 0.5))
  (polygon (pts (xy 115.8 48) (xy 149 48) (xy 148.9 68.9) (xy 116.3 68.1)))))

